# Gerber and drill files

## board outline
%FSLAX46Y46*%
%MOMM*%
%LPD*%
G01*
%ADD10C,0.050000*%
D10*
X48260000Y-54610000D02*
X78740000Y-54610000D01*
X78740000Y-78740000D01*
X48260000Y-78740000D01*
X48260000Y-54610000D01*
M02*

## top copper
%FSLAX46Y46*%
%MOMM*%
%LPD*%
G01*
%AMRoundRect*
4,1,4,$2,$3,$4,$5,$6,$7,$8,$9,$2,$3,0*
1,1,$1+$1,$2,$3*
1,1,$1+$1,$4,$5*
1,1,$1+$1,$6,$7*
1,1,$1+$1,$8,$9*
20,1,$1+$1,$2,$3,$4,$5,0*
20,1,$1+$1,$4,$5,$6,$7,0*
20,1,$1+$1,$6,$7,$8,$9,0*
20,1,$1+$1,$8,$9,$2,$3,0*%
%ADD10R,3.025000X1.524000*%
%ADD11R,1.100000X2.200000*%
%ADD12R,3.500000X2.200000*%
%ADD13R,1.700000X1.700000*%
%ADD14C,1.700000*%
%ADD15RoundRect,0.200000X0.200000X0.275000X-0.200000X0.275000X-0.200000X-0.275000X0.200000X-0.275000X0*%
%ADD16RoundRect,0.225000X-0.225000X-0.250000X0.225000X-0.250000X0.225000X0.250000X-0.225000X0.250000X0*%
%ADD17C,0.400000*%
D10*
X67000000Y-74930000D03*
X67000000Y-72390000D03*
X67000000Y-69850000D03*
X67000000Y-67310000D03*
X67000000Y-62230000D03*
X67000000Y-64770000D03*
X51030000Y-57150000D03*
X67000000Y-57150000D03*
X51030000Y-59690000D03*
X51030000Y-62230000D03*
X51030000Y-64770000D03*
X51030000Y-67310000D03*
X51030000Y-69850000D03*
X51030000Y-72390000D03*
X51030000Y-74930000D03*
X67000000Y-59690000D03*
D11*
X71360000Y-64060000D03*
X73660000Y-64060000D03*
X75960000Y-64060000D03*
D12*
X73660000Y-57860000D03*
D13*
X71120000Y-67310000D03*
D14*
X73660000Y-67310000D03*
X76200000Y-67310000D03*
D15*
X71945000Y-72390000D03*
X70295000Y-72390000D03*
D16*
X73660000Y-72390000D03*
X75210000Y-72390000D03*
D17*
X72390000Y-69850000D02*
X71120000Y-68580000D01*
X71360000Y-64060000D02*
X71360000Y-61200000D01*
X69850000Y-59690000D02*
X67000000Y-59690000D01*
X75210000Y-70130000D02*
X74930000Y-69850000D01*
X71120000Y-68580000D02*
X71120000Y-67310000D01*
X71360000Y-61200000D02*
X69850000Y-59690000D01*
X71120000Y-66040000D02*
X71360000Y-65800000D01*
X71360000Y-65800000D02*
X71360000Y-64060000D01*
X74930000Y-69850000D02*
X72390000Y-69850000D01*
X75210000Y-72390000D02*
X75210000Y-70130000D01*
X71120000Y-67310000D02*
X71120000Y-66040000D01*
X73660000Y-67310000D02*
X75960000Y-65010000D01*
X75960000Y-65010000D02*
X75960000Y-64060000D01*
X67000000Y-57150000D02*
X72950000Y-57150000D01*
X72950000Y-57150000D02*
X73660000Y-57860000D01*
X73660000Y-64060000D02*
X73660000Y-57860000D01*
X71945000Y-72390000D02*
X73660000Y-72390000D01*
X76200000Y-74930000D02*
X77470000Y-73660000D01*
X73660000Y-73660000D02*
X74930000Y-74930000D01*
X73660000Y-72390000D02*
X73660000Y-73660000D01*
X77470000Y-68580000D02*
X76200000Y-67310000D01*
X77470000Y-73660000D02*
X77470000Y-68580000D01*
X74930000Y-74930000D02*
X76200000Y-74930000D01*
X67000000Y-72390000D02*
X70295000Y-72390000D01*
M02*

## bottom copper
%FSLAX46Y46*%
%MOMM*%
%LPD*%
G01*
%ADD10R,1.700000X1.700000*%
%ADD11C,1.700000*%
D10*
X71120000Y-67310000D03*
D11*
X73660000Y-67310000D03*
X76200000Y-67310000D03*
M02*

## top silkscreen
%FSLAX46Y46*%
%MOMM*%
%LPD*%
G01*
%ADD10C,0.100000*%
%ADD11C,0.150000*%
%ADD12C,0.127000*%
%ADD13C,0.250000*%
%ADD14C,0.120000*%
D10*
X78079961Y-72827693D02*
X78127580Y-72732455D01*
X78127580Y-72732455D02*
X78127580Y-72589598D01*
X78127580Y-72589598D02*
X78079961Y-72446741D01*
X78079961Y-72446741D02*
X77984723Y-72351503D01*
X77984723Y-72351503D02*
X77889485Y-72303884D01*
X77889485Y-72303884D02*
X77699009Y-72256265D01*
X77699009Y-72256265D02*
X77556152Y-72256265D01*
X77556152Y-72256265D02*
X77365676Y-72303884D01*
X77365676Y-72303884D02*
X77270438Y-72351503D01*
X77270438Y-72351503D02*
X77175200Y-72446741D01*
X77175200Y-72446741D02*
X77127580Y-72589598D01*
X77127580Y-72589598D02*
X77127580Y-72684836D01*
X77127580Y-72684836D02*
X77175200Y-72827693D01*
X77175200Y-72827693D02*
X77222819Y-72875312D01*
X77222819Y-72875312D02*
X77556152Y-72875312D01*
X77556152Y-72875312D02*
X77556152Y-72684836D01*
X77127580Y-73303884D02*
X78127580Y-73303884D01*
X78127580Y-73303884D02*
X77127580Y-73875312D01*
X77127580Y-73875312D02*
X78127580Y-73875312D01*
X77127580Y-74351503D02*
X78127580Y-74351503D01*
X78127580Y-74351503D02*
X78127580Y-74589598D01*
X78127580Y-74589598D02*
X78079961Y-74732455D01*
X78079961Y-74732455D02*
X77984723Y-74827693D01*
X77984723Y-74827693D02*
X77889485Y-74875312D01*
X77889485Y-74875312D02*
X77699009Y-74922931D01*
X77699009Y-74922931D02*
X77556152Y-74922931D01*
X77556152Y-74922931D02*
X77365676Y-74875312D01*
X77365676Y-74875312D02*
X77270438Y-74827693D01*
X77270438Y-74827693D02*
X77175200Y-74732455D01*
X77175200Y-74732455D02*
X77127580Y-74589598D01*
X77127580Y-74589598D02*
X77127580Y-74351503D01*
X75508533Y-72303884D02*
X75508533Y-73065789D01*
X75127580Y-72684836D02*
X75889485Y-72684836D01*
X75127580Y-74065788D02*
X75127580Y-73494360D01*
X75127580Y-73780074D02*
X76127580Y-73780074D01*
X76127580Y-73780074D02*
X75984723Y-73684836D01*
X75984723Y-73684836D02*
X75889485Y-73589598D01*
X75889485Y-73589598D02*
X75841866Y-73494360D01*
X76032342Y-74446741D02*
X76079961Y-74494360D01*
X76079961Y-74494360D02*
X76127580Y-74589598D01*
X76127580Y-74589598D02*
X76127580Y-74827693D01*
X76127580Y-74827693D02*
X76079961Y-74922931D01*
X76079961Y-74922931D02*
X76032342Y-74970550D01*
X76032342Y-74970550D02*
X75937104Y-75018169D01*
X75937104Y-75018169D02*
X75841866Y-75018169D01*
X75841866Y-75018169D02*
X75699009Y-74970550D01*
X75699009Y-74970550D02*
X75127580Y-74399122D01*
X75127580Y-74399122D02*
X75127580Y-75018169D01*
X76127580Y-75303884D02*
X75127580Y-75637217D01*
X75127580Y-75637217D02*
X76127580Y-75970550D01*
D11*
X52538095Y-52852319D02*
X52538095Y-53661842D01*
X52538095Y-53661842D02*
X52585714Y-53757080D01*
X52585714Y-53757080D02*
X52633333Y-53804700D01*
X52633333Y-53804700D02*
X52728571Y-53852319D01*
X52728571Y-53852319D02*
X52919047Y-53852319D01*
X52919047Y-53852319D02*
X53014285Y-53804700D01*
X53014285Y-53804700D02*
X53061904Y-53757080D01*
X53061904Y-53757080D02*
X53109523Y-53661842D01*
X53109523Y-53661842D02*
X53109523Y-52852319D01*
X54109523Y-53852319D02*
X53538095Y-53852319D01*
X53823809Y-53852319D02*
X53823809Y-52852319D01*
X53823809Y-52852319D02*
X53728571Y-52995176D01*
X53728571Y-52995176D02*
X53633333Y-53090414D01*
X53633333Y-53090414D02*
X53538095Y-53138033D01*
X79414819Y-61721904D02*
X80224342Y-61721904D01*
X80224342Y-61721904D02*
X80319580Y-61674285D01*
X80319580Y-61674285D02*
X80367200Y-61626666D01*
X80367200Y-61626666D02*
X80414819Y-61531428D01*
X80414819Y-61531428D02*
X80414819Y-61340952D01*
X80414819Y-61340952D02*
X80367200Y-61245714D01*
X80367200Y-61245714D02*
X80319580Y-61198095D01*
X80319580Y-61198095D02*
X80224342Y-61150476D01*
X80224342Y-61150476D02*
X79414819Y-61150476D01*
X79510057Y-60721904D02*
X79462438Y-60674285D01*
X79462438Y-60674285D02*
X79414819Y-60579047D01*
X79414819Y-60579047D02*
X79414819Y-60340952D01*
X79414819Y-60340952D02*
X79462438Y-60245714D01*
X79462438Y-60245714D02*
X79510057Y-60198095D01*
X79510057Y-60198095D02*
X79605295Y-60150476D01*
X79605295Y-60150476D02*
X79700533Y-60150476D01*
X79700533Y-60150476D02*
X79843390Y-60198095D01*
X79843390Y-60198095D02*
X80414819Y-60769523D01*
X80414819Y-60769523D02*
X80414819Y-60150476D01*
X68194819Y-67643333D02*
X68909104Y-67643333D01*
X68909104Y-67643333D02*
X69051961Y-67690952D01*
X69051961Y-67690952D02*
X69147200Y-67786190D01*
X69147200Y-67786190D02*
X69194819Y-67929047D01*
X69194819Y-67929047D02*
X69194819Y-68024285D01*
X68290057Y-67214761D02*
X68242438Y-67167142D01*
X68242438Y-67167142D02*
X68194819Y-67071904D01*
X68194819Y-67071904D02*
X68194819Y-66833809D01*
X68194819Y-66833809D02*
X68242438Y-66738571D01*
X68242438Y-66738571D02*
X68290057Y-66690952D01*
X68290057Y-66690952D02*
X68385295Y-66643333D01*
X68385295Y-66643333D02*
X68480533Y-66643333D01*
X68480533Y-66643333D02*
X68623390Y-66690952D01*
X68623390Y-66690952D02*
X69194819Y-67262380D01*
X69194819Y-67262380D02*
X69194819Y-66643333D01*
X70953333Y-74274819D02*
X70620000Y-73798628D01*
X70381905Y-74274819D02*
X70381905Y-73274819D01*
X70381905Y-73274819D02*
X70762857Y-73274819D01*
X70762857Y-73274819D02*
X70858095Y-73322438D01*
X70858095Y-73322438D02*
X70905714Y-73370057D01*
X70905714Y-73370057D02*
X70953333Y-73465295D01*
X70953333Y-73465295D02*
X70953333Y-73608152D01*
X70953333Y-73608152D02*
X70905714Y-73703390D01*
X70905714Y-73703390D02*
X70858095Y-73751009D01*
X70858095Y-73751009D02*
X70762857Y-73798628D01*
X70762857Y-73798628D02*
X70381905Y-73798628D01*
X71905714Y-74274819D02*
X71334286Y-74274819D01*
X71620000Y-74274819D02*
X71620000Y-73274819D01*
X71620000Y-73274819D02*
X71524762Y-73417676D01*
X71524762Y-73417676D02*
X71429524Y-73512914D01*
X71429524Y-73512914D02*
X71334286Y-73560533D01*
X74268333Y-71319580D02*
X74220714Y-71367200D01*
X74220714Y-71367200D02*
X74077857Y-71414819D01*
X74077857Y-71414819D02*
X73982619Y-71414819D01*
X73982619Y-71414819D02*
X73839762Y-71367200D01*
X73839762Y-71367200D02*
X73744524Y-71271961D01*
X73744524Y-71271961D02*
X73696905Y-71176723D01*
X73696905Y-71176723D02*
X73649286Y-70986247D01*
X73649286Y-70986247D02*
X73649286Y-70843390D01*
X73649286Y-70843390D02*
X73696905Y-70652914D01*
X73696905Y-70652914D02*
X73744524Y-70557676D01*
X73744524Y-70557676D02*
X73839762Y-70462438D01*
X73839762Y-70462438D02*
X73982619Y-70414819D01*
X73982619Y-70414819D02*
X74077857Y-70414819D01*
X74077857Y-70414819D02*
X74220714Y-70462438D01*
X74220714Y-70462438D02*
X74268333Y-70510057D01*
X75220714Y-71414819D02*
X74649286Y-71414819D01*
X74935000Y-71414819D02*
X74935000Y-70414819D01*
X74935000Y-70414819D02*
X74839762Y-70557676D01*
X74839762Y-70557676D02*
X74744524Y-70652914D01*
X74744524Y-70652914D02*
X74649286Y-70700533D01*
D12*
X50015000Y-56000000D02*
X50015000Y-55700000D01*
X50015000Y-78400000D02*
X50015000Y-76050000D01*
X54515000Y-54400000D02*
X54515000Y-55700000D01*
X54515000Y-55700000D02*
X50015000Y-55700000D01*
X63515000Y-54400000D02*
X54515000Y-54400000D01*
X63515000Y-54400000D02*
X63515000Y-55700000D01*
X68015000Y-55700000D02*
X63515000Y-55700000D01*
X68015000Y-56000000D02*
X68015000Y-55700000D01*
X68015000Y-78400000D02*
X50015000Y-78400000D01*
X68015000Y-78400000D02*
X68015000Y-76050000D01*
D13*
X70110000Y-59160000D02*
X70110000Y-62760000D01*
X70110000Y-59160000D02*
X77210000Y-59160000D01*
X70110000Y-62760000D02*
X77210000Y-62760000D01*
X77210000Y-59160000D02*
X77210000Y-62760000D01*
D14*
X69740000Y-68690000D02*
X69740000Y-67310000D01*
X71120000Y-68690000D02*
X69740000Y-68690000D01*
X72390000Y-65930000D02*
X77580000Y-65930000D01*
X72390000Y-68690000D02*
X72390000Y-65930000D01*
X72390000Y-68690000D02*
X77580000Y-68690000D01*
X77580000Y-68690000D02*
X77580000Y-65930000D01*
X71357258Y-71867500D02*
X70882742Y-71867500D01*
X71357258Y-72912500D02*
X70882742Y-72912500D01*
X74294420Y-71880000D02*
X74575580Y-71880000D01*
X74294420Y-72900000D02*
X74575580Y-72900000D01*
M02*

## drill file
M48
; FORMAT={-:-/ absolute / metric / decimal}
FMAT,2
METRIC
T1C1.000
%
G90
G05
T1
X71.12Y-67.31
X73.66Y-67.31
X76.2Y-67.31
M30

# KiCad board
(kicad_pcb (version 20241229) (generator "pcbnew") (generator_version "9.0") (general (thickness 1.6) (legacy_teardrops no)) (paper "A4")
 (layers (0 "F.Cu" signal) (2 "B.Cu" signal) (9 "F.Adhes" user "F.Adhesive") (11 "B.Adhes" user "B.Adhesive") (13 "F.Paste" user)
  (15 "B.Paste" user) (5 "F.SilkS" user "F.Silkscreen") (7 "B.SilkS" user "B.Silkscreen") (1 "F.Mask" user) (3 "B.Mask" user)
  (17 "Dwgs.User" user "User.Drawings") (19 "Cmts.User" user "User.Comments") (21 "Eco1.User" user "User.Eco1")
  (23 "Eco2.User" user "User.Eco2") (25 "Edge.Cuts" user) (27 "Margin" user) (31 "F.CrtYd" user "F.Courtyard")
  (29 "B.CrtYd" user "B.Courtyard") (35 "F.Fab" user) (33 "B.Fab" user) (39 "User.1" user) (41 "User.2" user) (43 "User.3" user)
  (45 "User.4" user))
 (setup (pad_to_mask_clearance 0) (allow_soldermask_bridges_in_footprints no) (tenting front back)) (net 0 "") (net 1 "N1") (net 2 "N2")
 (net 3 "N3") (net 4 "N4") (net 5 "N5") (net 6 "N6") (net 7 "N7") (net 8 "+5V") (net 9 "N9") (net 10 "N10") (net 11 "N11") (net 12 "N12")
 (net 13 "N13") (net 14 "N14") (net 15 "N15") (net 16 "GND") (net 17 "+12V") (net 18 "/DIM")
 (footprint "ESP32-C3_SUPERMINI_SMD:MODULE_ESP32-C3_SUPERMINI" (layer "F.Cu") (at 59.015 67.05)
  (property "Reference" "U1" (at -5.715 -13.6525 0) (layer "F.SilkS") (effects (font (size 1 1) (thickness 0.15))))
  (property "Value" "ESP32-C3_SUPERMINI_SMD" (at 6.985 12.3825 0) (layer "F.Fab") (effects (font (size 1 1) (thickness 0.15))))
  (fp_line (start -9 -11.05) (end -9 -11.35) (stroke (width 0.127) (type solid)) (layer "F.SilkS"))
  (fp_line (start -9 11.35) (end -9 9) (stroke (width 0.127) (type solid)) (layer "F.SilkS"))
  (fp_line (start -4.5 -12.65) (end -4.5 -11.35) (stroke (width 0.127) (type solid)) (layer "F.SilkS"))
  (fp_line (start -4.5 -11.35) (end -9 -11.35) (stroke (width 0.127) (type solid)) (layer "F.SilkS"))
  (fp_line (start 4.5 -12.65) (end -4.5 -12.65) (stroke (width 0.127) (type solid)) (layer "F.SilkS"))
  (fp_line (start 4.5 -12.65) (end 4.5 -11.35) (stroke (width 0.127) (type solid)) (layer "F.SilkS"))
  (fp_line (start 9 -11.35) (end 4.5 -11.35) (stroke (width 0.127) (type solid)) (layer "F.SilkS"))
  (fp_line (start 9 -11.05) (end 9 -11.35) (stroke (width 0.127) (type solid)) (layer "F.SilkS"))
  (fp_line (start 9 11.35) (end -9 11.35) (stroke (width 0.127) (type solid)) (layer "F.SilkS"))
  (fp_line (start 9 11.35) (end 9 9) (stroke (width 0.127) (type solid)) (layer "F.SilkS"))
  (pad "0" smd rect (at 7.985 7.88) (size 3.025 1.524) (layers "F.Cu" "F.Mask" "F.Paste") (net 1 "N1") (solder_mask_margin 0.102))
  (pad "1" smd rect (at 7.985 5.34) (size 3.025 1.524) (layers "F.Cu" "F.Mask" "F.Paste") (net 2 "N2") (solder_mask_margin 0.102))
  (pad "2" smd rect (at 7.985 2.8) (size 3.025 1.524) (layers "F.Cu" "F.Mask" "F.Paste") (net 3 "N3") (solder_mask_margin 0.102))
  (pad "3" smd rect (at 7.985 0.26) (size 3.025 1.524) (layers "F.Cu" "F.Mask" "F.Paste") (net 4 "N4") (solder_mask_margin 0.102))
  (pad "3.3" smd rect (at 7.985 -4.82) (size 3.025 1.524) (layers "F.Cu" "F.Mask" "F.Paste") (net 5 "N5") (solder_mask_margin 0.102))
  (pad "4" smd rect (at 7.985 -2.28) (size 3.025 1.524) (layers "F.Cu" "F.Mask" "F.Paste") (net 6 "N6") (solder_mask_margin 0.102))
  (pad "5" smd rect (at -7.985 -9.9) (size 3.025 1.524) (layers "F.Cu" "F.Mask" "F.Paste") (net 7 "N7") (solder_mask_margin 0.102))
  (pad "5V" smd rect (at 7.985 -9.9) (size 3.025 1.524) (layers "F.Cu" "F.Mask" "F.Paste") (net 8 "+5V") (solder_mask_margin 0.102))
  (pad "6" smd rect (at -7.985 -7.36) (size 3.025 1.524) (layers "F.Cu" "F.Mask" "F.Paste") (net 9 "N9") (solder_mask_margin 0.102))
  (pad "7" smd rect (at -7.985 -4.82) (size 3.025 1.524) (layers "F.Cu" "F.Mask" "F.Paste") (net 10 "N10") (solder_mask_margin 0.102))
  (pad "8" smd rect (at -7.985 -2.28) (size 3.025 1.524) (layers "F.Cu" "F.Mask" "F.Paste") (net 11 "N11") (solder_mask_margin 0.102))
  (pad "9" smd rect (at -7.985 0.26) (size 3.025 1.524) (layers "F.Cu" "F.Mask" "F.Paste") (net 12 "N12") (solder_mask_margin 0.102))
  (pad "10" smd rect (at -7.985 2.8) (size 3.025 1.524) (layers "F.Cu" "F.Mask" "F.Paste") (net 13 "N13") (solder_mask_margin 0.102))
  (pad "20" smd rect (at -7.985 5.34) (size 3.025 1.524) (layers "F.Cu" "F.Mask" "F.Paste") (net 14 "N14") (solder_mask_margin 0.102))
  (pad "21" smd rect (at -7.985 7.88) (size 3.025 1.524) (layers "F.Cu" "F.Mask" "F.Paste") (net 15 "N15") (solder_mask_margin 0.102))
  (pad "G" smd rect (at 7.985 -7.36) (size 3.025 1.524) (layers "F.Cu" "F.Mask" "F.Paste") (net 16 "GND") (solder_mask_margin 0.102)))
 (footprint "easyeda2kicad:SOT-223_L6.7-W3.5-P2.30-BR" (layer "F.Cu") (at 73.66 60.96 -90)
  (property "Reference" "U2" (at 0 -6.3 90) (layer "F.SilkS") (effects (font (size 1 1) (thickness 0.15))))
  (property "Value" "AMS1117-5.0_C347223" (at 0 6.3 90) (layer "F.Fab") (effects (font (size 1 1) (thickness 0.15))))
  (fp_line (start -1.8 3.55) (end 1.8 3.55) (stroke (width 0.25) (type solid)) (layer "F.SilkS"))
  (fp_line (start -1.8 3.55) (end -1.8 -3.55) (stroke (width 0.25) (type solid)) (layer "F.SilkS"))
  (fp_line (start 1.8 3.55) (end 1.8 -3.55) (stroke (width 0.25) (type solid)) (layer "F.SilkS"))
  (fp_line (start -1.8 -3.55) (end 1.8 -3.55) (stroke (width 0.25) (type solid)) (layer "F.SilkS"))
  (pad "1" smd rect (at 3.1 2.3) (size 1.1 2.2) (layers "F.Cu" "F.Mask" "F.Paste") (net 16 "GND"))
  (pad "2" smd rect (at 3.1 0) (size 1.1 2.2) (layers "F.Cu" "F.Mask" "F.Paste") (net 8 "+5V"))
  (pad "3" smd rect (at 3.1 -2.3) (size 1.1 2.2) (layers "F.Cu" "F.Mask" "F.Paste") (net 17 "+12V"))
  (pad "4" smd rect (at -3.1 0 270) (size 2.2 3.5) (layers "F.Cu" "F.Mask" "F.Paste") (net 8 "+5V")))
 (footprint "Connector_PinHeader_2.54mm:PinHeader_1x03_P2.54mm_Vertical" (layer "F.Cu") (at 71.12 67.31 90)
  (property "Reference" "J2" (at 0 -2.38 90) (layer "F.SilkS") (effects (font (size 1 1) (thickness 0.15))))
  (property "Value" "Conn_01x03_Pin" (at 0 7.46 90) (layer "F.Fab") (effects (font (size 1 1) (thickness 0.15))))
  (fp_line (start -1.38 -1.38) (end 0 -1.38) (stroke (width 0.12) (type solid)) (layer "F.SilkS"))
  (fp_line (start -1.38 0) (end -1.38 -1.38) (stroke (width 0.12) (type solid)) (layer "F.SilkS"))
  (fp_line (start 1.38 1.27) (end 1.38 6.46) (stroke (width 0.12) (type solid)) (layer "F.SilkS"))
  (fp_line (start -1.38 1.27) (end 1.38 1.27) (stroke (width 0.12) (type solid)) (layer "F.SilkS"))
  (fp_line (start -1.38 1.27) (end -1.38 6.46) (stroke (width 0.12) (type solid)) (layer "F.SilkS"))
  (fp_line (start -1.38 6.46) (end 1.38 6.46) (stroke (width 0.12) (type solid)) (layer "F.SilkS"))
  (pad "1" thru_hole rect (at 0 0 90) (size 1.7 1.7) (drill 1) (layers "*.Cu" "*.Mask") (remove_unused_layers no) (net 16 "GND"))
  (pad "2" thru_hole circle (at 0 2.54 90) (size 1.7 1.7) (drill 1) (layers "*.Cu" "*.Mask") (remove_unused_layers no) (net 17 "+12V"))
  (pad "3" thru_hole circle (at 0 5.08 90) (size 1.7 1.7) (drill 1) (layers "*.Cu" "*.Mask") (remove_unused_layers no) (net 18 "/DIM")))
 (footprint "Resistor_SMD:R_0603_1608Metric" (layer "F.Cu") (at 71.12 72.39 180)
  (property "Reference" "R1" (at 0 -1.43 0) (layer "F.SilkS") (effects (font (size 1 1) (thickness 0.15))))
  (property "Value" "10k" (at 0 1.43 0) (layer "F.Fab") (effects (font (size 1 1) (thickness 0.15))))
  (fp_line (start -0.237258 0.5225) (end 0.237258 0.5225) (stroke (width 0.12) (type solid)) (layer "F.SilkS"))
  (fp_line (start -0.237258 -0.5225) (end 0.237258 -0.5225) (stroke (width 0.12) (type solid)) (layer "F.SilkS"))
  (pad "1" smd roundrect (at -0.825 0 180) (size 0.8 0.95) (layers "F.Cu" "F.Mask" "F.Paste") (roundrect_rratio 0.25) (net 18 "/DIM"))
  (pad "2" smd roundrect (at 0.825 0 180) (size 0.8 0.95) (layers "F.Cu" "F.Mask" "F.Paste") (roundrect_rratio 0.25) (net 2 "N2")))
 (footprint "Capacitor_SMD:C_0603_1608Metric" (layer "F.Cu") (at 74.435 72.39)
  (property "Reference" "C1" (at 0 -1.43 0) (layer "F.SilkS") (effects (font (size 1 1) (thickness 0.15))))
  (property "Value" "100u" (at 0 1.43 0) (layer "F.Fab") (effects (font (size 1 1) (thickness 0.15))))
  (fp_line (start -0.14058 -0.51) (end 0.14058 -0.51) (stroke (width 0.12) (type solid)) (layer "F.SilkS"))
  (fp_line (start -0.14058 0.51) (end 0.14058 0.51) (stroke (width 0.12) (type solid)) (layer "F.SilkS"))
  (pad "1" smd roundrect (at -0.775 0) (size 0.9 0.95) (layers "F.Cu" "F.Mask" "F.Paste") (roundrect_rratio 0.25) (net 18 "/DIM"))
  (pad "2" smd roundrect (at 0.775 0) (size 0.9 0.95) (layers "F.Cu" "F.Mask" "F.Paste") (roundrect_rratio 0.25) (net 16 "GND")))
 (gr_rect (start 48.26 54.61) (end 78.74 78.74) (stroke (width 0.05) (type default)) (fill no) (layer "Edge.Cuts"))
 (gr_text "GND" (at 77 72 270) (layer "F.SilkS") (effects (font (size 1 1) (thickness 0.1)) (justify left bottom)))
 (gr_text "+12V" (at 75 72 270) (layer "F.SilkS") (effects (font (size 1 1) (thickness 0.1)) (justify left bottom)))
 (segment (start 72.39 69.85) (end 71.12 68.58) (width 0.4) (layer "F.Cu") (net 16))
 (segment (start 71.36 64.06) (end 71.36 61.2) (width 0.4) (layer "F.Cu") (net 16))
 (segment (start 69.85 59.69) (end 67 59.69) (width 0.4) (layer "F.Cu") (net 16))
 (segment (start 75.21 70.13) (end 74.93 69.85) (width 0.4) (layer "F.Cu") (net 16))
 (segment (start 71.12 68.58) (end 71.12 67.31) (width 0.4) (layer "F.Cu") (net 16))
 (segment (start 71.36 61.2) (end 69.85 59.69) (width 0.4) (layer "F.Cu") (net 16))
 (segment (start 71.12 66.04) (end 71.36 65.8) (width 0.4) (layer "F.Cu") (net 16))
 (segment (start 71.36 65.8) (end 71.36 64.06) (width 0.4) (layer "F.Cu") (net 16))
 (segment (start 74.93 69.85) (end 72.39 69.85) (width 0.4) (layer "F.Cu") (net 16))
 (segment (start 75.21 72.39) (end 75.21 70.13) (width 0.4) (layer "F.Cu") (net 16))
 (segment (start 71.12 67.31) (end 71.12 66.04) (width 0.4) (layer "F.Cu") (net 16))
 (segment (start 73.66 67.31) (end 75.96 65.01) (width 0.4) (layer "F.Cu") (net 17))
 (segment (start 75.96 65.01) (end 75.96 64.06) (width 0.4) (layer "F.Cu") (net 17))
 (segment (start 67 57.15) (end 72.95 57.15) (width 0.4) (layer "F.Cu") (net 8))
 (segment (start 72.95 57.15) (end 73.66 57.86) (width 0.4) (layer "F.Cu") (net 8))
 (segment (start 73.66 64.06) (end 73.66 57.86) (width 0.4) (layer "F.Cu") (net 8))
 (segment (start 71.945 72.39) (end 73.66 72.39) (width 0.4) (layer "F.Cu") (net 18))
 (segment (start 76.2 74.93) (end 77.47 73.66) (width 0.4) (layer "F.Cu") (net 18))
 (segment (start 73.66 73.66) (end 74.93 74.93) (width 0.4) (layer "F.Cu") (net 18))
 (segment (start 73.66 72.39) (end 73.66 73.66) (width 0.4) (layer "F.Cu") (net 18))
 (segment (start 77.47 68.58) (end 76.2 67.31) (width 0.4) (layer "F.Cu") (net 18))
 (segment (start 77.47 73.66) (end 77.47 68.58) (width 0.4) (layer "F.Cu") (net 18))
 (segment (start 74.93 74.93) (end 76.2 74.93) (width 0.4) (layer "F.Cu") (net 18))
 (segment (start 67 72.39) (end 70.295 72.39) (width 0.4) (layer "F.Cu") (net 2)))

